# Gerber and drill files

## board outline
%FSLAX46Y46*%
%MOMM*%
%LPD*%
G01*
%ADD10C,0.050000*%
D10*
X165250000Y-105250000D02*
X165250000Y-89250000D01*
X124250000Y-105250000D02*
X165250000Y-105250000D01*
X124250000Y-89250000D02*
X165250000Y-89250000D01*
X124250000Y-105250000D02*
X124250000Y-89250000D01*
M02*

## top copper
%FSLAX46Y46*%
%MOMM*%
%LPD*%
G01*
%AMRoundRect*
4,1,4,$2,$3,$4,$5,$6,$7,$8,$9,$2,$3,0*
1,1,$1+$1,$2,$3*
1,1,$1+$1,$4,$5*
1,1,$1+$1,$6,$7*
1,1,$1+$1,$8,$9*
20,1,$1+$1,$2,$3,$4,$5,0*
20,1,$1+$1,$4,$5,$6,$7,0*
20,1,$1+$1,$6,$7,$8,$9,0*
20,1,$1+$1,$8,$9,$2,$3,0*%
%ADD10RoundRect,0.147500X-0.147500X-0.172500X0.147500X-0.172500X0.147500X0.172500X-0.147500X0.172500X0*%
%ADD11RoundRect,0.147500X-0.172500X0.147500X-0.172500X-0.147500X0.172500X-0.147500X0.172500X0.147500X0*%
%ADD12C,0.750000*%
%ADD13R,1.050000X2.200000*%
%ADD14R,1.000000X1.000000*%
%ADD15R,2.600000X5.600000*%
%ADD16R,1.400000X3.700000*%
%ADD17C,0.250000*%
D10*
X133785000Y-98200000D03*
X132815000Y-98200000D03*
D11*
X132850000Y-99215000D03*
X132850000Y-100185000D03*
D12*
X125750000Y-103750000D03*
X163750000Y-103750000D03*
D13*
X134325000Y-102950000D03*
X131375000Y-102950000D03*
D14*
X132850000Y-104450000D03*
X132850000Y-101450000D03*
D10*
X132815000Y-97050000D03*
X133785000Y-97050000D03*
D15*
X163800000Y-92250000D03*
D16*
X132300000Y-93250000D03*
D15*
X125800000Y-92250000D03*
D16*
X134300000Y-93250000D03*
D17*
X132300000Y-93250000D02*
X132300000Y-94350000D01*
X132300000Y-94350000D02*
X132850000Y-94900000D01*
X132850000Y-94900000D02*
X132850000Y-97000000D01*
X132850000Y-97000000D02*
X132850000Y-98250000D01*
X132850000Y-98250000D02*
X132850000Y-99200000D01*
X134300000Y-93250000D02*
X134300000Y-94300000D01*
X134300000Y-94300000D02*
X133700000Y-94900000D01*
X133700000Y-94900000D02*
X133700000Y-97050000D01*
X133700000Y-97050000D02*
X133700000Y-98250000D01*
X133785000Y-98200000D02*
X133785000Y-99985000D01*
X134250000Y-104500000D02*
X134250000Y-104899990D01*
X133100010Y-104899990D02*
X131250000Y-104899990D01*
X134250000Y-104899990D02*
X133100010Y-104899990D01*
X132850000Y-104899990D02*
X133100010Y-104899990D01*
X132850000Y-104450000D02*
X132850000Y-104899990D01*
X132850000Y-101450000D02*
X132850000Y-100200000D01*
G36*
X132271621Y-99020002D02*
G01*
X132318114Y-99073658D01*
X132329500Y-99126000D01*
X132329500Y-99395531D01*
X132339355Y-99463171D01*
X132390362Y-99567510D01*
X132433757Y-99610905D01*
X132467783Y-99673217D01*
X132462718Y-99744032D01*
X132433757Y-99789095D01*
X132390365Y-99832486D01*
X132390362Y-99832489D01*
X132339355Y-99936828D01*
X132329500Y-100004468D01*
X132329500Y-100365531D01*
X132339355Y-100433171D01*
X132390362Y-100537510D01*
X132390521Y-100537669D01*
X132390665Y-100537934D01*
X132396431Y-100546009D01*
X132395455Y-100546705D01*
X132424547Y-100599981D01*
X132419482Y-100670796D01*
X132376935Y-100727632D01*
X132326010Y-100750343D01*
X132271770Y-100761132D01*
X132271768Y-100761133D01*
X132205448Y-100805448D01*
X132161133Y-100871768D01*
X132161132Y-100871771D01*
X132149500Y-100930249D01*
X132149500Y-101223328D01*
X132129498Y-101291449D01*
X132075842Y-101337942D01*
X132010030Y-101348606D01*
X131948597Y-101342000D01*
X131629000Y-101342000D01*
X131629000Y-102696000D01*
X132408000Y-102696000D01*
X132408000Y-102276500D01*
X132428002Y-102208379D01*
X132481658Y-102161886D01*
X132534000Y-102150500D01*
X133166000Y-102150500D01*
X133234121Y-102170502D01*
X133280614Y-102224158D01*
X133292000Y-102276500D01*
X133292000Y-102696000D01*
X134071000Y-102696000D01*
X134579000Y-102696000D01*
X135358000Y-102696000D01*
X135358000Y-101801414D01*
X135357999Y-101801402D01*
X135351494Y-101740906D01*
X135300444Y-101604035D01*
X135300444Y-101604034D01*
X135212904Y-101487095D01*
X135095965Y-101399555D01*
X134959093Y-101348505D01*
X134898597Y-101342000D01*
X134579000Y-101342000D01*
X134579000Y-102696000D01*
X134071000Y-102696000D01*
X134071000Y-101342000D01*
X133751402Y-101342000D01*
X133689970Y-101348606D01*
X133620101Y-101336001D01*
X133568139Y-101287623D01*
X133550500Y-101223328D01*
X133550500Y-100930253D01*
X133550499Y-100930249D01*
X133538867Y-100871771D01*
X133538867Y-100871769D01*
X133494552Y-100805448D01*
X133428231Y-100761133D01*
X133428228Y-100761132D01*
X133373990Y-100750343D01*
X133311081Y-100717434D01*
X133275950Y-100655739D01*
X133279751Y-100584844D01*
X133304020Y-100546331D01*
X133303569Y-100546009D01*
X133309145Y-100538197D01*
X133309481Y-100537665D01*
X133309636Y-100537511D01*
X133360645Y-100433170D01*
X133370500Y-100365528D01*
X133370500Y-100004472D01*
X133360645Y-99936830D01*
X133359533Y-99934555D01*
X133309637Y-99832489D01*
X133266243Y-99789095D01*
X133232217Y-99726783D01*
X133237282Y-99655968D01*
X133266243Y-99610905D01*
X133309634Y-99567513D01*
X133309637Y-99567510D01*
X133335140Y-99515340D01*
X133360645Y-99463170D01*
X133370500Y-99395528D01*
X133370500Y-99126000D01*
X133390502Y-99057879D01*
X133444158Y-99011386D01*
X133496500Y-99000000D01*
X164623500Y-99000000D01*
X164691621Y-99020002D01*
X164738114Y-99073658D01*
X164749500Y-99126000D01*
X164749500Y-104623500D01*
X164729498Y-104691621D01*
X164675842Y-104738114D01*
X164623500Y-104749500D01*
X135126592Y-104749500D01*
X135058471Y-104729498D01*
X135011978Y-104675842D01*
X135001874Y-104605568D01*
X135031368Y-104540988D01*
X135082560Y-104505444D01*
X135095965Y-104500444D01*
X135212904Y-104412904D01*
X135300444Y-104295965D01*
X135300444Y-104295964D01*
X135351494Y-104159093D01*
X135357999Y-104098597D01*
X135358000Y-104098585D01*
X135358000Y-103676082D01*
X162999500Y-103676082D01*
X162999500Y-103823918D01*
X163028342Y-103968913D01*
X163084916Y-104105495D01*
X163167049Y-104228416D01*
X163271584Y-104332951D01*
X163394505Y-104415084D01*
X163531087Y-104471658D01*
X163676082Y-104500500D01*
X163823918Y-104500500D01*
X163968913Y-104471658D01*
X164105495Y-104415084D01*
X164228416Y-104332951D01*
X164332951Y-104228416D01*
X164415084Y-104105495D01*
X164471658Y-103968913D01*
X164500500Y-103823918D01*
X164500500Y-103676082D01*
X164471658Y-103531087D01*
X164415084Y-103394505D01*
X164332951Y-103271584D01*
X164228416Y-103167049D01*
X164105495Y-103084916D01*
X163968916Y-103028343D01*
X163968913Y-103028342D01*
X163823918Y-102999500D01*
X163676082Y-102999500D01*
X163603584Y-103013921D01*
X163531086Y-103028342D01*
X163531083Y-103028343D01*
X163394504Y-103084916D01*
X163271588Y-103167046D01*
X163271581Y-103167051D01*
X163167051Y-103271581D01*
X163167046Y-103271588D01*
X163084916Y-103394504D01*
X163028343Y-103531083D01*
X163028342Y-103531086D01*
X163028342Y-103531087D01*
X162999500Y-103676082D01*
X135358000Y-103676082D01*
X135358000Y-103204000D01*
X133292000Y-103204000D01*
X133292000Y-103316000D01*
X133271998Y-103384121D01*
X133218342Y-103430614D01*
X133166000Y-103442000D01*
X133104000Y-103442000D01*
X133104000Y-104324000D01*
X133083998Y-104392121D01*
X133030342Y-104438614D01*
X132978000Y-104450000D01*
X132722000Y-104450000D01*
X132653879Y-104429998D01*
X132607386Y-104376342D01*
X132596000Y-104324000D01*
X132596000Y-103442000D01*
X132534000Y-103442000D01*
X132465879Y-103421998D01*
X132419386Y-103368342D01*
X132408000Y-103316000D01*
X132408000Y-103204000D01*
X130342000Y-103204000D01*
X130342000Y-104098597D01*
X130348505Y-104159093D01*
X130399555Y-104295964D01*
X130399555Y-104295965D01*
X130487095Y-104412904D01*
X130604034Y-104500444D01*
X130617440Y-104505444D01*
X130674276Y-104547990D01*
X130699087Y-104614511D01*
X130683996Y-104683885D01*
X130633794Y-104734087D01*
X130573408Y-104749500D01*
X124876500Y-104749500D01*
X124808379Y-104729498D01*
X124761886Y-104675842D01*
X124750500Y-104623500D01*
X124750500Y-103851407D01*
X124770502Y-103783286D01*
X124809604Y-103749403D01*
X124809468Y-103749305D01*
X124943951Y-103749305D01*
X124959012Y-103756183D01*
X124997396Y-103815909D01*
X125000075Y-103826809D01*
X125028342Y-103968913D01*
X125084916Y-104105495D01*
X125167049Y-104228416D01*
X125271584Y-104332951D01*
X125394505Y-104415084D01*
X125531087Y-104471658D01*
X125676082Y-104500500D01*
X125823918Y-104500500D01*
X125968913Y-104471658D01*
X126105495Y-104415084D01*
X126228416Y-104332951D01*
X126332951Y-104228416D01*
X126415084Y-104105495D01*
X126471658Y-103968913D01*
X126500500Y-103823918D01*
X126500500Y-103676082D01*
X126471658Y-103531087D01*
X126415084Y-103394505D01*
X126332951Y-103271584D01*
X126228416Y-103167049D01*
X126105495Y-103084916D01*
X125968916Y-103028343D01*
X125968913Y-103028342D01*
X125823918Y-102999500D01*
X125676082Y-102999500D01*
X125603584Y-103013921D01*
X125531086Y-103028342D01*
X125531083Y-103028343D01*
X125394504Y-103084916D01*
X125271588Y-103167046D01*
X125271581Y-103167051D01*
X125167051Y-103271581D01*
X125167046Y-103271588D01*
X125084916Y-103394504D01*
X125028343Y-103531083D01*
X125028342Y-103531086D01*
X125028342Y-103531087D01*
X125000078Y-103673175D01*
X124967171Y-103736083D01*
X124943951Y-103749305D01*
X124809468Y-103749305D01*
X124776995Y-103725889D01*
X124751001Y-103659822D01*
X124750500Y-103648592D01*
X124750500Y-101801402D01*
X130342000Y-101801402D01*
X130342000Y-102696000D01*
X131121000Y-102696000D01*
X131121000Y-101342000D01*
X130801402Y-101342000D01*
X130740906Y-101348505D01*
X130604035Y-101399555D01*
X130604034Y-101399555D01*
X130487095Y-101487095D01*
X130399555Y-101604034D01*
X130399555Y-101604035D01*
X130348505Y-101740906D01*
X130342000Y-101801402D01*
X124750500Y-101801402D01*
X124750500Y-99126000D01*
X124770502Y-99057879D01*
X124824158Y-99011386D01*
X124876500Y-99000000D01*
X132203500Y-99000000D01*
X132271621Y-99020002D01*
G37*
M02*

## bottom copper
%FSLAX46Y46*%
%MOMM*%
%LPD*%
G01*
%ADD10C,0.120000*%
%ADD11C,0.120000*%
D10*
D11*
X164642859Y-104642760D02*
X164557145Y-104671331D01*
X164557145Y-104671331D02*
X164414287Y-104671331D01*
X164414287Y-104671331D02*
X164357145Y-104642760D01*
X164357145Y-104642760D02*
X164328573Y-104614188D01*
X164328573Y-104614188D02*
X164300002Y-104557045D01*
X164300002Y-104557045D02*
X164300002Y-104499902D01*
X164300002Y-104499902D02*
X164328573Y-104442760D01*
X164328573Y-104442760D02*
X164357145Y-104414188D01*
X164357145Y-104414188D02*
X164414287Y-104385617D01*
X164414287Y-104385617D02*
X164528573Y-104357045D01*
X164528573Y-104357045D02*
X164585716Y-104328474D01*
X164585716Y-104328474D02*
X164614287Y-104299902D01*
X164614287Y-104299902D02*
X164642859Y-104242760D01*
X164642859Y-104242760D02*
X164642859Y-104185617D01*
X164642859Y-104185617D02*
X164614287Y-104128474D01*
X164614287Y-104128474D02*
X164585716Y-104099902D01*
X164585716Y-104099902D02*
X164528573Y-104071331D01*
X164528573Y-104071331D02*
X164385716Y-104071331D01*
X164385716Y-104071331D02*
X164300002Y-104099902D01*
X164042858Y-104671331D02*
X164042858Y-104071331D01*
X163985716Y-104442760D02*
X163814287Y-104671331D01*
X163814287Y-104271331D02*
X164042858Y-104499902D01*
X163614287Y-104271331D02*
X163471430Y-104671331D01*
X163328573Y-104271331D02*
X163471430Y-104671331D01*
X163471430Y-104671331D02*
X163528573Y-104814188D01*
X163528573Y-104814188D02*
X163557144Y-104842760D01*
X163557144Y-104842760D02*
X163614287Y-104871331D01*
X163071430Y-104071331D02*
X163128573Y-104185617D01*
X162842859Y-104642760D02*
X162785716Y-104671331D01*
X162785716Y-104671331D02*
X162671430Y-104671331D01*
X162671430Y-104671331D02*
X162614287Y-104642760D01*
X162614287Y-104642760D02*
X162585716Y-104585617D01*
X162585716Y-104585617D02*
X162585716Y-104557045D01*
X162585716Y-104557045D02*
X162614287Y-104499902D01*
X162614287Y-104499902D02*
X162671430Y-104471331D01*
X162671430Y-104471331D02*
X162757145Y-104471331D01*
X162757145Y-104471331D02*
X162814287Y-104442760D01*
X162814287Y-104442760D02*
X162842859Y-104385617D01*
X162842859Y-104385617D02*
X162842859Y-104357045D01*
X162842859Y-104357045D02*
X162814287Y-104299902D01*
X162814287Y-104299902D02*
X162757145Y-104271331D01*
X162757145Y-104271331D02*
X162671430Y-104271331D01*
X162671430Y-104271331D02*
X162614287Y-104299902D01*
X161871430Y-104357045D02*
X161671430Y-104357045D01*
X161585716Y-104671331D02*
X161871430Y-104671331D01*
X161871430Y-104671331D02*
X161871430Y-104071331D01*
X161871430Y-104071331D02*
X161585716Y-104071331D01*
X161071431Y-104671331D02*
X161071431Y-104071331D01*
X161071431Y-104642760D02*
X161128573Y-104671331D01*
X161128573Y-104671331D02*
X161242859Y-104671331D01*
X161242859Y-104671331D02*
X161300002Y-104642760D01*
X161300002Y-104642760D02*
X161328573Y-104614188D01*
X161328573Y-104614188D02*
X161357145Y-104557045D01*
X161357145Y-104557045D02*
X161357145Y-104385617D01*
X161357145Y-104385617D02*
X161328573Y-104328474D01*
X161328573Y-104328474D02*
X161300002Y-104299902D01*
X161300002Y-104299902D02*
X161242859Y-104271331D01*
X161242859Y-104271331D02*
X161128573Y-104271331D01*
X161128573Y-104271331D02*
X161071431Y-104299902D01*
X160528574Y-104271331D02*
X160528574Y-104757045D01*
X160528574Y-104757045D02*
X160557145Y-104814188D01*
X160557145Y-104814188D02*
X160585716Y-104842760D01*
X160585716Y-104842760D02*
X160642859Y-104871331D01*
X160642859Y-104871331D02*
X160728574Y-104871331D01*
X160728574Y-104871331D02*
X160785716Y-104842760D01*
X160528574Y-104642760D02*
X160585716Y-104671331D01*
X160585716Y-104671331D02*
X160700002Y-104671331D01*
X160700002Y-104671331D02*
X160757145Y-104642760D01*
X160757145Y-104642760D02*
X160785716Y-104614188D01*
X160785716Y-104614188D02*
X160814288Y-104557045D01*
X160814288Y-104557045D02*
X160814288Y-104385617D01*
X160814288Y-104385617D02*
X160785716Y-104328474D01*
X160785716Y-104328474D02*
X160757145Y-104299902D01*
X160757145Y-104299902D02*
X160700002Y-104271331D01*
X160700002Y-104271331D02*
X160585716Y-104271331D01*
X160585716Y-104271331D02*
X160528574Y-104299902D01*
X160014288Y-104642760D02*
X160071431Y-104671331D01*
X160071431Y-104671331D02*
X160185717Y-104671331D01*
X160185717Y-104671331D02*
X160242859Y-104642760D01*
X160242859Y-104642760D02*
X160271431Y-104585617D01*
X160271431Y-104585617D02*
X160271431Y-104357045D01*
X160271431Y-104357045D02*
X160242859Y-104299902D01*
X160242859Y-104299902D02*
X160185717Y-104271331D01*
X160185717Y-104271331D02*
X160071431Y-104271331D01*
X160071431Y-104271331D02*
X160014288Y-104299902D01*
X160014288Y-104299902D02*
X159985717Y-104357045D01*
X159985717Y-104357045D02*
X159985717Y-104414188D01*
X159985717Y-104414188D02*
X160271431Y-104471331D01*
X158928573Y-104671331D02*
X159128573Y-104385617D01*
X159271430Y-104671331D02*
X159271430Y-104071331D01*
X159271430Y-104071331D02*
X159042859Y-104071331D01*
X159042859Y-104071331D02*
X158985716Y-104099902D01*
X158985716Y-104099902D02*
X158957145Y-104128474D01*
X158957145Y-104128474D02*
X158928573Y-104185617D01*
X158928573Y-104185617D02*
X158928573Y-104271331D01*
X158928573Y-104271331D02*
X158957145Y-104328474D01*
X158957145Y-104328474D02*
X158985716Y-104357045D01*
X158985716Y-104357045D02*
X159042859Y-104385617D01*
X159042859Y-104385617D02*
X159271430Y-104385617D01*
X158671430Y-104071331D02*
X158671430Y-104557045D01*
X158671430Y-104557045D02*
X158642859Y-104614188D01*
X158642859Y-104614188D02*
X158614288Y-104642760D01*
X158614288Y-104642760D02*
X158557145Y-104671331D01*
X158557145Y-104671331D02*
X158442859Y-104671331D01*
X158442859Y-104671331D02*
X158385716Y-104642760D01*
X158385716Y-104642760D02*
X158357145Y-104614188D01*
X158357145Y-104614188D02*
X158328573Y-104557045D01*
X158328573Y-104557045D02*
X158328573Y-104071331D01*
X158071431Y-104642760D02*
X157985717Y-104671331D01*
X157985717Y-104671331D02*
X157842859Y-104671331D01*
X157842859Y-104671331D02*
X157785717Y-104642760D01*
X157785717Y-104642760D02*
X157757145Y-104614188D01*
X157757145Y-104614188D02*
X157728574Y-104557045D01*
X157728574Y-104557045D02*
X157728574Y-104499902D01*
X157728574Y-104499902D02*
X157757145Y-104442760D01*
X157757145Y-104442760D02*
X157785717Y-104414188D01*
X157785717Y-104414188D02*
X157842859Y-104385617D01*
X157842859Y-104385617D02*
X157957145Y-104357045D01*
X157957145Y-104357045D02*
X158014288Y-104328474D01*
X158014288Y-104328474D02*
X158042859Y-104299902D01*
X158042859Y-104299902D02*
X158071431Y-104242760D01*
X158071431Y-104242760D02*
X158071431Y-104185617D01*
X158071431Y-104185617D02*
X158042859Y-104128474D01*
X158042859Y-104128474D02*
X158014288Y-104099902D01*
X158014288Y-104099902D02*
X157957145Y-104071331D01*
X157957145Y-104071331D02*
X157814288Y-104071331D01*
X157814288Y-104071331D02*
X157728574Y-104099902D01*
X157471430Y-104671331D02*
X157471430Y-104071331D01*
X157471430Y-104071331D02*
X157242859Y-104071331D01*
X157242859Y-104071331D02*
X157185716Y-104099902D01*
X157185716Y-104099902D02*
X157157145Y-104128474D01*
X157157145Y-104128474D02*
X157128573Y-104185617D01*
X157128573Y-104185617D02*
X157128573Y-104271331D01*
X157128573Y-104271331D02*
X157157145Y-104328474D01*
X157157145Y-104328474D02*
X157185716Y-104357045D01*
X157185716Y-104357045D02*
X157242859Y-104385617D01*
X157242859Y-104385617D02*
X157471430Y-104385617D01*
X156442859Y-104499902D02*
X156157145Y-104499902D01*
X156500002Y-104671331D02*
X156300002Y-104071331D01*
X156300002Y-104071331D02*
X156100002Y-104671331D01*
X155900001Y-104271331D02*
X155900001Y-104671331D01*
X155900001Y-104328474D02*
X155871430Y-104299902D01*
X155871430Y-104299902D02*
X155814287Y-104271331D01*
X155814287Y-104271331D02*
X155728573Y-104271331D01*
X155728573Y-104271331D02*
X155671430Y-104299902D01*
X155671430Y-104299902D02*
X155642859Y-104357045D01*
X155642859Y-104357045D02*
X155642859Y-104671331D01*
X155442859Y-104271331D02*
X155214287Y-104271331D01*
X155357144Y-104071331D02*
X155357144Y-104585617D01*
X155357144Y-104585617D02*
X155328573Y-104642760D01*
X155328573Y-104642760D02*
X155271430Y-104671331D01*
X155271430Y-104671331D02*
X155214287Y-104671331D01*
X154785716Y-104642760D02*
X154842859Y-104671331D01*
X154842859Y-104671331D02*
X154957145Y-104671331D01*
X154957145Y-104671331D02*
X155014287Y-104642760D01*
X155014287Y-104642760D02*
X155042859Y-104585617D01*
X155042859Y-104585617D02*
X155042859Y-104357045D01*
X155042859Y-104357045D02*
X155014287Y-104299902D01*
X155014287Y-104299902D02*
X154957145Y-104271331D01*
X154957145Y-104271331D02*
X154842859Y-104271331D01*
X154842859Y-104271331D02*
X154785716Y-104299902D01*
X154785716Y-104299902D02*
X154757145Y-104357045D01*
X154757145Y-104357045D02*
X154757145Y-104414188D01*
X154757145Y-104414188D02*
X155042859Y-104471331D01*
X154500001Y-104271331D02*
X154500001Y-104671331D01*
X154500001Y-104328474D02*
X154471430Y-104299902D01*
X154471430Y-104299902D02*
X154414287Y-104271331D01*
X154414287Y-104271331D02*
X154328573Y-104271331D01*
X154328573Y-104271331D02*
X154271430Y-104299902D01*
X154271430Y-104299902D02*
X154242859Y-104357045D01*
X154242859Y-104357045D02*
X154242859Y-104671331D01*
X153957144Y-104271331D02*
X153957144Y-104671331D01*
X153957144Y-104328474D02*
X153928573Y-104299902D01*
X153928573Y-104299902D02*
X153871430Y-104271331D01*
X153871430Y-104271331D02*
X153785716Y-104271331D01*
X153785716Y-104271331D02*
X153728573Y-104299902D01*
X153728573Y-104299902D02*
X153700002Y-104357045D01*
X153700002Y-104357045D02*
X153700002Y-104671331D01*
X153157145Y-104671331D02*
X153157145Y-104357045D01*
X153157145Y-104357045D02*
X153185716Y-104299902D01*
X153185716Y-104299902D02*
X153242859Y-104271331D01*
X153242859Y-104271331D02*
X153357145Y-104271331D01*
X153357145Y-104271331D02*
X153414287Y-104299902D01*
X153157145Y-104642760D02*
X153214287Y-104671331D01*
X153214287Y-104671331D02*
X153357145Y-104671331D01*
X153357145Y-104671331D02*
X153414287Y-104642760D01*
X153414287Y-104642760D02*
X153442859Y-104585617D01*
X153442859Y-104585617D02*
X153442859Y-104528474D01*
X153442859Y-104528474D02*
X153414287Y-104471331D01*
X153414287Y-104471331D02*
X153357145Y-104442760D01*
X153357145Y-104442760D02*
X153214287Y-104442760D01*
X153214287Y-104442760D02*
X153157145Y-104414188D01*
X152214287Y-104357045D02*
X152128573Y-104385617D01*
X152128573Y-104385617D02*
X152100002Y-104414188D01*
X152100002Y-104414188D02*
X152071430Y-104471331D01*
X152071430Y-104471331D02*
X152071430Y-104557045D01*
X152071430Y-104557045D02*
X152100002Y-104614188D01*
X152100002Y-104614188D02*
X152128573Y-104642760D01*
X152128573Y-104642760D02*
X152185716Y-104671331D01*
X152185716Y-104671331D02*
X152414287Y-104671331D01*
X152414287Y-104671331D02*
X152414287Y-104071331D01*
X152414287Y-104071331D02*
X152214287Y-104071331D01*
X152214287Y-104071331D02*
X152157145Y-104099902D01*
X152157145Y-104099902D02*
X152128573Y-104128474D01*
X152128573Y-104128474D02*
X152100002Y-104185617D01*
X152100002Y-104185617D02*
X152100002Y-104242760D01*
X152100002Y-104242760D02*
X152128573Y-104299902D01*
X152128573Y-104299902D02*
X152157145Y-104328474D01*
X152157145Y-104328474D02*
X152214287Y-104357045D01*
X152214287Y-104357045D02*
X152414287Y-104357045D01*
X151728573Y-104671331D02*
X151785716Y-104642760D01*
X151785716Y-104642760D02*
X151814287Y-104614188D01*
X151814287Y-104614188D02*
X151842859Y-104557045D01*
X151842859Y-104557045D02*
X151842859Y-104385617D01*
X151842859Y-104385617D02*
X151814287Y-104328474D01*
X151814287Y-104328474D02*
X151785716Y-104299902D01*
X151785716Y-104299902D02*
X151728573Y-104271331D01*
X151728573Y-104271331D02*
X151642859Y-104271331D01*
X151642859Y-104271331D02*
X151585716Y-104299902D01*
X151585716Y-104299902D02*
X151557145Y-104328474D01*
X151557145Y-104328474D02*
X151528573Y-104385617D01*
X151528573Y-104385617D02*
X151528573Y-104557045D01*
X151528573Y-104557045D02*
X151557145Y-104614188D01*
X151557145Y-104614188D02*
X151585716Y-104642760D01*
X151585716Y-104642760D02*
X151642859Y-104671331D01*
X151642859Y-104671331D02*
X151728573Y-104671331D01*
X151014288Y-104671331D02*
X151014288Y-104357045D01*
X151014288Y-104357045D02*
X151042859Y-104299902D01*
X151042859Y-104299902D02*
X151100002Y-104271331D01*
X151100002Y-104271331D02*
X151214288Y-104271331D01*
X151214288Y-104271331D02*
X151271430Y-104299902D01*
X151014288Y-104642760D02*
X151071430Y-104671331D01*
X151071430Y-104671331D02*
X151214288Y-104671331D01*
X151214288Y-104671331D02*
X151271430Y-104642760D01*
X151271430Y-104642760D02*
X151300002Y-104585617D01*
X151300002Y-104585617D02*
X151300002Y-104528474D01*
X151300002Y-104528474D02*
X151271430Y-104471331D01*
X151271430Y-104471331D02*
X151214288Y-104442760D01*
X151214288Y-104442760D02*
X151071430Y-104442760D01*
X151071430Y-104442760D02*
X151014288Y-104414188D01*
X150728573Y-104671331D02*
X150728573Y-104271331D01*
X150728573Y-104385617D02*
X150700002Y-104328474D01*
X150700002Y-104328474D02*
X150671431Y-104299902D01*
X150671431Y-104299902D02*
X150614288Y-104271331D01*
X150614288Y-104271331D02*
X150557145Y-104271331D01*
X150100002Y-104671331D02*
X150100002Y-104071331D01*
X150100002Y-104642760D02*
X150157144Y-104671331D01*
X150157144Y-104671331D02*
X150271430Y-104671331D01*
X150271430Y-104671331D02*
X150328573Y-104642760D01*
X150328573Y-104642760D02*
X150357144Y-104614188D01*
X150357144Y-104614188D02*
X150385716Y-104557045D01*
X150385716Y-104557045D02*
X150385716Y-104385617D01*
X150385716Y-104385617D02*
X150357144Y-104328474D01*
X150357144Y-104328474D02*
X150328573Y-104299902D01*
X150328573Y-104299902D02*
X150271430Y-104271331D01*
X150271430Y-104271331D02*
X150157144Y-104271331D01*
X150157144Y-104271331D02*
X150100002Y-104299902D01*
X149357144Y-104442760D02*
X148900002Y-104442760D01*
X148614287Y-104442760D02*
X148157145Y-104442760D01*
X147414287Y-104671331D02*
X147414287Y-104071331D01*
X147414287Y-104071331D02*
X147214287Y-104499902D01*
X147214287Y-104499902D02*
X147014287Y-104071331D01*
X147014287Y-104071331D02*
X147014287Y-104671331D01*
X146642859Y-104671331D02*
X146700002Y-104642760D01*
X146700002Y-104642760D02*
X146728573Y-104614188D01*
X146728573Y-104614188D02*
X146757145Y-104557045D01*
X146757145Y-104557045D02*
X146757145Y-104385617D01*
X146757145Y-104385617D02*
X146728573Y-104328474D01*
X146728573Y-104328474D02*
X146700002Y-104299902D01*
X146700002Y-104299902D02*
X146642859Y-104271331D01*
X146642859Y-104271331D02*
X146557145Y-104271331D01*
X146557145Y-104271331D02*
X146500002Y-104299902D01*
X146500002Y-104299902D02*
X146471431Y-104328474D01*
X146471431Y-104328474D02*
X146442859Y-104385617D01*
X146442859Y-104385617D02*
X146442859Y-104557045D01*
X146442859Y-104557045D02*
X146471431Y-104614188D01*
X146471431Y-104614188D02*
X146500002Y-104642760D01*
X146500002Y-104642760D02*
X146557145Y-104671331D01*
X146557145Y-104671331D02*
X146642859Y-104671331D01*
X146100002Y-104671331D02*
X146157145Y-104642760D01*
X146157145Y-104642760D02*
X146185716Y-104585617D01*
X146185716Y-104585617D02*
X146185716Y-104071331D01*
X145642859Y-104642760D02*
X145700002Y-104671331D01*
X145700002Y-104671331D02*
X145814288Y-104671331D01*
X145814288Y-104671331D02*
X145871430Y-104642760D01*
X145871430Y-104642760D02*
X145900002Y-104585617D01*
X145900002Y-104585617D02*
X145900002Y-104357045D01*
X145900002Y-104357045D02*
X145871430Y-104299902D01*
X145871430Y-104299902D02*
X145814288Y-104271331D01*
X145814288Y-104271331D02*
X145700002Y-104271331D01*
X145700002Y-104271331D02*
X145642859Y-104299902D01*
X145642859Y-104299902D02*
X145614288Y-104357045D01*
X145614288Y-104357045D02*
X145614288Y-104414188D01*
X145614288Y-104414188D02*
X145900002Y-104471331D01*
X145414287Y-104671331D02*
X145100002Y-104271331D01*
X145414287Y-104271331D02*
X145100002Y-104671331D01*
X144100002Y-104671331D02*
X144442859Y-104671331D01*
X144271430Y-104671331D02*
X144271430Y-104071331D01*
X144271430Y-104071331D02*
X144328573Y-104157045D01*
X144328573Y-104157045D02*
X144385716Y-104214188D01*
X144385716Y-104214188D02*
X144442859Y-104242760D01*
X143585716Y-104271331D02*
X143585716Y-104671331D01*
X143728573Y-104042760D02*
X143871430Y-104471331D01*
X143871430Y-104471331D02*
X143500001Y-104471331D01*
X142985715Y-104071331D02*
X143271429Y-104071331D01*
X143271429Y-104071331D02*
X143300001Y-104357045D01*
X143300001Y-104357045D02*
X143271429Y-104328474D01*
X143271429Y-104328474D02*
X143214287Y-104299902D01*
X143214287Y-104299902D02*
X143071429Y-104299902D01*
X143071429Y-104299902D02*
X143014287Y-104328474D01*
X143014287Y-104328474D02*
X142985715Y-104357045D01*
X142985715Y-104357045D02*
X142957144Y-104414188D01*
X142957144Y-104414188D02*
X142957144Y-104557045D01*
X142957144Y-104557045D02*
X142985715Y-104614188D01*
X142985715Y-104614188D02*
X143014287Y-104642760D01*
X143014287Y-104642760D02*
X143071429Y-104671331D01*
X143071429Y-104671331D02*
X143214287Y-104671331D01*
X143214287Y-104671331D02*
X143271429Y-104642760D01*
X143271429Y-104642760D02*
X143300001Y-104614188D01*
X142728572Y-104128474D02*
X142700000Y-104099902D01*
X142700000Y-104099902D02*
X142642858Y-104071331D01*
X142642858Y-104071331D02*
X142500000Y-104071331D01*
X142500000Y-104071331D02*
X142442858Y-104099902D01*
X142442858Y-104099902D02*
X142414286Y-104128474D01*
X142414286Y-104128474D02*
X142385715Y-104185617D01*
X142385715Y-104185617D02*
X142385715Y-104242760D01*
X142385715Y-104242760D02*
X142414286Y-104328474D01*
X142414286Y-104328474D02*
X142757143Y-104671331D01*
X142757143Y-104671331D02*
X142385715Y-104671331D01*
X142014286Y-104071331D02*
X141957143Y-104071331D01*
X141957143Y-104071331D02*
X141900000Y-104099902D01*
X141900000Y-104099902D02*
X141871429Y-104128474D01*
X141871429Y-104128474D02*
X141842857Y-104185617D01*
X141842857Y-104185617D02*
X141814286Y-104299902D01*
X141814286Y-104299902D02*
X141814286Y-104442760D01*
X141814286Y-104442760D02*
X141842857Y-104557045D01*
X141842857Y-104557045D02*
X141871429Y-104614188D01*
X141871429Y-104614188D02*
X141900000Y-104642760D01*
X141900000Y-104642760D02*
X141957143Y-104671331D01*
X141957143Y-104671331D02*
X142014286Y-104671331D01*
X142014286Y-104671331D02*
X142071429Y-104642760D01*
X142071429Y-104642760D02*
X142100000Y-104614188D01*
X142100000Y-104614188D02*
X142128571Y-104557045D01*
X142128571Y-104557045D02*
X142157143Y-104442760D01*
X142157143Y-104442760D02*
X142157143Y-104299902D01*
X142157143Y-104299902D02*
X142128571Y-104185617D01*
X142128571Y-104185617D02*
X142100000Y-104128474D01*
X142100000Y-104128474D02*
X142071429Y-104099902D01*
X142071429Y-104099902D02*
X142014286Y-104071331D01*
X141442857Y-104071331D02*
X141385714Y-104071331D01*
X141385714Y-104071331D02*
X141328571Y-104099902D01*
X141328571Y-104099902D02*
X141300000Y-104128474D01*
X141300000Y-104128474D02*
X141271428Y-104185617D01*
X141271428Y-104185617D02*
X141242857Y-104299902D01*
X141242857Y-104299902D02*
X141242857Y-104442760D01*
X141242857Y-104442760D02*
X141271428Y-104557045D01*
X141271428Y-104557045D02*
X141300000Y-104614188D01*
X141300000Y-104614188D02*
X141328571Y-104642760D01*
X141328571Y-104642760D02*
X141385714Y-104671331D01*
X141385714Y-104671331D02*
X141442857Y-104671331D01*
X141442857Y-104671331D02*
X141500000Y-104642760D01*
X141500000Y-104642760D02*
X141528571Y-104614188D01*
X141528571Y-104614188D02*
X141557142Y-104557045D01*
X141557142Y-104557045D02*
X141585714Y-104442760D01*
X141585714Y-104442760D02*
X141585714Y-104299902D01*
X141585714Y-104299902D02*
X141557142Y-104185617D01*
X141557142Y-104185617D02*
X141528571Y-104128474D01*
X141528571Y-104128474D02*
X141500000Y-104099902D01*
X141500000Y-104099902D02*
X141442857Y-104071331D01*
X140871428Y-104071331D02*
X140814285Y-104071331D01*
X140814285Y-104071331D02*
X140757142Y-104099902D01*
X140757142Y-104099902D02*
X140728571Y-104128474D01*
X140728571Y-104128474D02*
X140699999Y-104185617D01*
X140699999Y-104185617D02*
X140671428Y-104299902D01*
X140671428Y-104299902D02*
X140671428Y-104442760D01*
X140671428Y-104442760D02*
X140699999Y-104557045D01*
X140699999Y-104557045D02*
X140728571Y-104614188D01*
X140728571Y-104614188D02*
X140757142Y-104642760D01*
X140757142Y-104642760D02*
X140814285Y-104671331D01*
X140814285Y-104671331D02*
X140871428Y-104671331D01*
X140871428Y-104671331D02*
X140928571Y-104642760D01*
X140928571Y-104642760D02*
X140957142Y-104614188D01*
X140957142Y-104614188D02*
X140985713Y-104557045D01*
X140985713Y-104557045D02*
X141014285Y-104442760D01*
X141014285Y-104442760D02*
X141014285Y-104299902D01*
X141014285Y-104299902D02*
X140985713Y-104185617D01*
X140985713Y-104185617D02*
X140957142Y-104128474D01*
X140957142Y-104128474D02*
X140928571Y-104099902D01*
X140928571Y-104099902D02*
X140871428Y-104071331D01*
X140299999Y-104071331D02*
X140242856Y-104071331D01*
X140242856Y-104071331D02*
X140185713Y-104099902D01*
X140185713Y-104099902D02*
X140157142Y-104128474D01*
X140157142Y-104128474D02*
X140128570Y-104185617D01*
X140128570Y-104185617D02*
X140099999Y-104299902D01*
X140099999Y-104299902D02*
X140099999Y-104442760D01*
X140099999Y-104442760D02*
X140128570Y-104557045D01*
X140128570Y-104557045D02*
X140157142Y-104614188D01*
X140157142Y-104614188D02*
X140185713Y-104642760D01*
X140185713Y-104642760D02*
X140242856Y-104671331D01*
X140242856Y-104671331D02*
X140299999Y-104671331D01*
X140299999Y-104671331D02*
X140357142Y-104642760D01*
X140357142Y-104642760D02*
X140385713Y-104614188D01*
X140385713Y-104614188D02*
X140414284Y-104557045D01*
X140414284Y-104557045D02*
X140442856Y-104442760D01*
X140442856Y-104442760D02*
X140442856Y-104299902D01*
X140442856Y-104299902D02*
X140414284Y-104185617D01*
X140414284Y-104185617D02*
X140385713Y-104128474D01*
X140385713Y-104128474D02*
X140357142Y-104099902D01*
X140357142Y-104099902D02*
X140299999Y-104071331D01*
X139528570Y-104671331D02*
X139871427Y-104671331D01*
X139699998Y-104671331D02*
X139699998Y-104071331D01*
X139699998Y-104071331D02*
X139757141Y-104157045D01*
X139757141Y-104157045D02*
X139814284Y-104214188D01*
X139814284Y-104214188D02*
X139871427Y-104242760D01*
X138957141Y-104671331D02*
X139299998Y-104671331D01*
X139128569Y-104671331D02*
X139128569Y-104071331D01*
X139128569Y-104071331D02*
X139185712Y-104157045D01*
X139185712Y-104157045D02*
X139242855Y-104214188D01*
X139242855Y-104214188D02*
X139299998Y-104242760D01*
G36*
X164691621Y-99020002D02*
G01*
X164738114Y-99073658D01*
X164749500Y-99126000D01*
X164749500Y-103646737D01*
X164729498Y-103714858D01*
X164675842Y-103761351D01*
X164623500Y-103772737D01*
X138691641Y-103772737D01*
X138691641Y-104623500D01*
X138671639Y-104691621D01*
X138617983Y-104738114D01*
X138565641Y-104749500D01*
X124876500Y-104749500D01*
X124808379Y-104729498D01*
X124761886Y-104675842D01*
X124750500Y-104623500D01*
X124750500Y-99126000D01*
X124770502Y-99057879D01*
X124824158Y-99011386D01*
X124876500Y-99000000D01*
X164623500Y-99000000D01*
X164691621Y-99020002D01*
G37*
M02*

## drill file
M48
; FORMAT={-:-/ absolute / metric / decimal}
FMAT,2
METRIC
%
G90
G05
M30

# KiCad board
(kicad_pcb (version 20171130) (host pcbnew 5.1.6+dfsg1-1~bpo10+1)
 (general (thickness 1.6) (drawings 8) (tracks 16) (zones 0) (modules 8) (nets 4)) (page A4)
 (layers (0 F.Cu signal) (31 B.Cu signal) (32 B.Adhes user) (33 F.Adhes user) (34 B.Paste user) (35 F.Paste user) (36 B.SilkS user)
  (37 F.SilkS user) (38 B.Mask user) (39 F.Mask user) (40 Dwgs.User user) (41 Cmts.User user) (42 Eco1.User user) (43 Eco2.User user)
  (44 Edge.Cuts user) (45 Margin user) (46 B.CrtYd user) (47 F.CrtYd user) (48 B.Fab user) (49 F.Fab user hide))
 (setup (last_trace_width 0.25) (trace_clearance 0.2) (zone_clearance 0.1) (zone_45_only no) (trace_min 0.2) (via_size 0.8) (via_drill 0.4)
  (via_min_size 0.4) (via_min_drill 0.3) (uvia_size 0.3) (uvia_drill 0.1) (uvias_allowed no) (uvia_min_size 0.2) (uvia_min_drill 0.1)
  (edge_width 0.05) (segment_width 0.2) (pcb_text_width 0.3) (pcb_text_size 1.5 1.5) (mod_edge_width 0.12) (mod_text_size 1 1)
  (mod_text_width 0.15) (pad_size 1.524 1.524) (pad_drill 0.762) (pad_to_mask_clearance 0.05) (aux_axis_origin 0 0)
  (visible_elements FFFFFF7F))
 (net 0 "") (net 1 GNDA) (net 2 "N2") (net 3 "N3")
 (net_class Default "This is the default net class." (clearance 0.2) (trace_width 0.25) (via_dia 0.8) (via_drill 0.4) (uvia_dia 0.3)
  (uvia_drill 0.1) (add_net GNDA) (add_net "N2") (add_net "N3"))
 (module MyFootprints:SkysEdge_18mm (layer F.Cu) (at 151.6 101.6)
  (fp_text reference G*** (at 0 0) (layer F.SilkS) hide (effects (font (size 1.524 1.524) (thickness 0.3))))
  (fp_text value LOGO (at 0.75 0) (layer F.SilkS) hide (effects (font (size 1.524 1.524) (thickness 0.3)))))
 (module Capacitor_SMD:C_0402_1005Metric (layer F.Cu) (at 133.3 98.2)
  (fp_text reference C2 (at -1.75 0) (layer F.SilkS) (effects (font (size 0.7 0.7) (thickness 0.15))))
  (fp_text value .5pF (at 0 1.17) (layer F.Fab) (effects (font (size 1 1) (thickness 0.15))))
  (pad 2 smd roundrect (at 0.485 0) (size 0.59 0.64) (layers F.Cu F.Paste F.Mask) (roundrect_rratio 0.25) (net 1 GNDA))
  (pad 1 smd roundrect (at -0.485 0) (size 0.59 0.64) (layers F.Cu F.Paste F.Mask) (roundrect_rratio 0.25) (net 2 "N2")))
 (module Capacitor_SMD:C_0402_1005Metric (layer F.Cu) (at 132.85 99.7 270)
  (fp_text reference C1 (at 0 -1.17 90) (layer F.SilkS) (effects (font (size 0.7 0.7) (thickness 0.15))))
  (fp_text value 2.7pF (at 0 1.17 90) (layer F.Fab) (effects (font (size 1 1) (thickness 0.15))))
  (pad 1 smd roundrect (at -0.485 0 270) (size 0.59 0.64) (layers F.Cu F.Paste F.Mask) (roundrect_rratio 0.25) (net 2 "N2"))
  (pad 2 smd roundrect (at 0.485 0 270) (size 0.59 0.64) (layers F.Cu F.Paste F.Mask) (roundrect_rratio 0.25) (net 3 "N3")))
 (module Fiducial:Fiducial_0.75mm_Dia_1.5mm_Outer (layer F.Cu) (at 125.75 103.75)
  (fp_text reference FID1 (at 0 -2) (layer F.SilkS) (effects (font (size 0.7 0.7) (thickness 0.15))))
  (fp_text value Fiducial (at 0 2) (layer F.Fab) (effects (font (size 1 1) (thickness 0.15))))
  (pad "" smd circle (at 0 0) (size 0.75 0.75) (layers F.Cu F.Mask) (solder_mask_margin 0.375) (clearance 0.375)))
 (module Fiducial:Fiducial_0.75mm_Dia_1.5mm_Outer (layer F.Cu) (at 163.75 103.75)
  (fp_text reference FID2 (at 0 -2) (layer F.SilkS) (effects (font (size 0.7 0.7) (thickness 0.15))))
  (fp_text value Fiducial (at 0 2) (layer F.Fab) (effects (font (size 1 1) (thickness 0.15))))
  (pad "" smd circle (at 0 0) (size 0.75 0.75) (layers F.Cu F.Mask) (solder_mask_margin 0.375) (clearance 0.375)))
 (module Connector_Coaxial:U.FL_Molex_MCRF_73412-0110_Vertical (layer F.Cu) (at 132.85 102.95 180)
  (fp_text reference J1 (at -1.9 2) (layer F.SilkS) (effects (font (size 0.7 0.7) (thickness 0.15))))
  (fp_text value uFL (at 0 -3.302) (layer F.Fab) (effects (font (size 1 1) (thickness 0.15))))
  (pad 2 smd rect (at -1.475 0 180) (size 1.05 2.2) (layers F.Cu F.Paste F.Mask) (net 1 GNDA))
  (pad 2 smd rect (at 1.475 0 180) (size 1.05 2.2) (layers F.Cu F.Paste F.Mask) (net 1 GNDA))
  (pad 2 smd rect (at 0 -1.5 180) (size 1 1) (layers F.Cu F.Paste F.Mask) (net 1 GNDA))
  (pad 1 smd rect (at 0 1.5 180) (size 1 1) (layers F.Cu F.Paste F.Mask) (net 3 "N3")))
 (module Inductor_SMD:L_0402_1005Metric (layer F.Cu) (at 133.3 97.05)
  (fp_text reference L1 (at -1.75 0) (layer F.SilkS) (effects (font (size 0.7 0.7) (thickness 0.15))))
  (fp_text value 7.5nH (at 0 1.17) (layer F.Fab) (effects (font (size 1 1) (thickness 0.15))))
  (pad 1 smd roundrect (at -0.485 0) (size 0.59 0.64) (layers F.Cu F.Paste F.Mask) (roundrect_rratio 0.25) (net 2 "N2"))
  (pad 2 smd roundrect (at 0.485 0) (size 0.59 0.64) (layers F.Cu F.Paste F.Mask) (roundrect_rratio 0.25) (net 1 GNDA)))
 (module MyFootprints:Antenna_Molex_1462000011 (layer F.Cu) (at 145.3 92.25)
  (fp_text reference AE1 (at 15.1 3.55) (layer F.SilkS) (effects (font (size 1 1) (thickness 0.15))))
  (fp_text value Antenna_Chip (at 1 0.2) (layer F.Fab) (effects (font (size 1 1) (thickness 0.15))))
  (pad "" smd rect (at 18.5 0) (size 2.6 5.6) (layers F.Cu F.Paste F.Mask))
  (pad 1 smd rect (at -13 1) (size 1.4 3.7) (layers F.Cu F.Paste F.Mask) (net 2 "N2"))
  (pad "" smd rect (at -19.5 0) (size 2.6 5.6) (layers F.Cu F.Paste F.Mask))
  (pad 2 smd rect (at -11 1) (size 1.4 3.7) (layers F.Cu F.Paste F.Mask) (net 1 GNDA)))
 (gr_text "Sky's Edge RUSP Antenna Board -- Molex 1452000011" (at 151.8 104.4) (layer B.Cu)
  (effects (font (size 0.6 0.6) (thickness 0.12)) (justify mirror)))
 (gr_line (start 165.25 105.25) (end 165.25 89.25) (layer Edge.Cuts) (width 0.05))
 (gr_line (start 124.25 105.25) (end 165.25 105.25) (layer Edge.Cuts) (width 0.05))
 (gr_line (start 124.25 89.25) (end 165.25 89.25) (layer Edge.Cuts) (width 0.05))
 (gr_line (start 124.25 105.25) (end 124.25 89.25) (layer Edge.Cuts) (width 0.05))
 (segment (start 132.3 93.25) (end 132.3 94.35) (width 0.25) (layer F.Cu) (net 2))
 (segment (start 132.3 94.35) (end 132.85 94.9) (width 0.25) (layer F.Cu) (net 2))
 (segment (start 132.85 94.9) (end 132.85 97) (width 0.25) (layer F.Cu) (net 2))
 (segment (start 132.85 97) (end 132.85 98.25) (width 0.25) (layer F.Cu) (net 2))
 (segment (start 132.85 98.25) (end 132.85 99.2) (width 0.25) (layer F.Cu) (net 2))
 (segment (start 134.3 93.25) (end 134.3 94.3) (width 0.25) (layer F.Cu) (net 1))
 (segment (start 134.3 94.3) (end 133.7 94.9) (width 0.25) (layer F.Cu) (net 1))
 (segment (start 133.7 94.9) (end 133.7 97.05) (width 0.25) (layer F.Cu) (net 1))
 (segment (start 133.7 97.05) (end 133.7 98.25) (width 0.25) (layer F.Cu) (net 1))
 (segment (start 133.785 98.2) (end 133.785 99.985) (width 0.25) (layer F.Cu) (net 1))
 (segment (start 134.25 104.5) (end 134.25 104.89999) (width 0.25) (layer F.Cu) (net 1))
 (segment (start 133.10001 104.89999) (end 131.25 104.89999) (width 0.25) (layer F.Cu) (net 1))
 (segment (start 134.25 104.89999) (end 133.10001 104.89999) (width 0.25) (layer F.Cu) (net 1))
 (segment (start 132.85 104.89999) (end 133.10001 104.89999) (width 0.25) (layer F.Cu) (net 1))
 (segment (start 132.85 104.45) (end 132.85 104.89999) (width 0.25) (layer F.Cu) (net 1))
 (segment (start 132.85 101.45) (end 132.85 100.2) (width 0.25) (layer F.Cu) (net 3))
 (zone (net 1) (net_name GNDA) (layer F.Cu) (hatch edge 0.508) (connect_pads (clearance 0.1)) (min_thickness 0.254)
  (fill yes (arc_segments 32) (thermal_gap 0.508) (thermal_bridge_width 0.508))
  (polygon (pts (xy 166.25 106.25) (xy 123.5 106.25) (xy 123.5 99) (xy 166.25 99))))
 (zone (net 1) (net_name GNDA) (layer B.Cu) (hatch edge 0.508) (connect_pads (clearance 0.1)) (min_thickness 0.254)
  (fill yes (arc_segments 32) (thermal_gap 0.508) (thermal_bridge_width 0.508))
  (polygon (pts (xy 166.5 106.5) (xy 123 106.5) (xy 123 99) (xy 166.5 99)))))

